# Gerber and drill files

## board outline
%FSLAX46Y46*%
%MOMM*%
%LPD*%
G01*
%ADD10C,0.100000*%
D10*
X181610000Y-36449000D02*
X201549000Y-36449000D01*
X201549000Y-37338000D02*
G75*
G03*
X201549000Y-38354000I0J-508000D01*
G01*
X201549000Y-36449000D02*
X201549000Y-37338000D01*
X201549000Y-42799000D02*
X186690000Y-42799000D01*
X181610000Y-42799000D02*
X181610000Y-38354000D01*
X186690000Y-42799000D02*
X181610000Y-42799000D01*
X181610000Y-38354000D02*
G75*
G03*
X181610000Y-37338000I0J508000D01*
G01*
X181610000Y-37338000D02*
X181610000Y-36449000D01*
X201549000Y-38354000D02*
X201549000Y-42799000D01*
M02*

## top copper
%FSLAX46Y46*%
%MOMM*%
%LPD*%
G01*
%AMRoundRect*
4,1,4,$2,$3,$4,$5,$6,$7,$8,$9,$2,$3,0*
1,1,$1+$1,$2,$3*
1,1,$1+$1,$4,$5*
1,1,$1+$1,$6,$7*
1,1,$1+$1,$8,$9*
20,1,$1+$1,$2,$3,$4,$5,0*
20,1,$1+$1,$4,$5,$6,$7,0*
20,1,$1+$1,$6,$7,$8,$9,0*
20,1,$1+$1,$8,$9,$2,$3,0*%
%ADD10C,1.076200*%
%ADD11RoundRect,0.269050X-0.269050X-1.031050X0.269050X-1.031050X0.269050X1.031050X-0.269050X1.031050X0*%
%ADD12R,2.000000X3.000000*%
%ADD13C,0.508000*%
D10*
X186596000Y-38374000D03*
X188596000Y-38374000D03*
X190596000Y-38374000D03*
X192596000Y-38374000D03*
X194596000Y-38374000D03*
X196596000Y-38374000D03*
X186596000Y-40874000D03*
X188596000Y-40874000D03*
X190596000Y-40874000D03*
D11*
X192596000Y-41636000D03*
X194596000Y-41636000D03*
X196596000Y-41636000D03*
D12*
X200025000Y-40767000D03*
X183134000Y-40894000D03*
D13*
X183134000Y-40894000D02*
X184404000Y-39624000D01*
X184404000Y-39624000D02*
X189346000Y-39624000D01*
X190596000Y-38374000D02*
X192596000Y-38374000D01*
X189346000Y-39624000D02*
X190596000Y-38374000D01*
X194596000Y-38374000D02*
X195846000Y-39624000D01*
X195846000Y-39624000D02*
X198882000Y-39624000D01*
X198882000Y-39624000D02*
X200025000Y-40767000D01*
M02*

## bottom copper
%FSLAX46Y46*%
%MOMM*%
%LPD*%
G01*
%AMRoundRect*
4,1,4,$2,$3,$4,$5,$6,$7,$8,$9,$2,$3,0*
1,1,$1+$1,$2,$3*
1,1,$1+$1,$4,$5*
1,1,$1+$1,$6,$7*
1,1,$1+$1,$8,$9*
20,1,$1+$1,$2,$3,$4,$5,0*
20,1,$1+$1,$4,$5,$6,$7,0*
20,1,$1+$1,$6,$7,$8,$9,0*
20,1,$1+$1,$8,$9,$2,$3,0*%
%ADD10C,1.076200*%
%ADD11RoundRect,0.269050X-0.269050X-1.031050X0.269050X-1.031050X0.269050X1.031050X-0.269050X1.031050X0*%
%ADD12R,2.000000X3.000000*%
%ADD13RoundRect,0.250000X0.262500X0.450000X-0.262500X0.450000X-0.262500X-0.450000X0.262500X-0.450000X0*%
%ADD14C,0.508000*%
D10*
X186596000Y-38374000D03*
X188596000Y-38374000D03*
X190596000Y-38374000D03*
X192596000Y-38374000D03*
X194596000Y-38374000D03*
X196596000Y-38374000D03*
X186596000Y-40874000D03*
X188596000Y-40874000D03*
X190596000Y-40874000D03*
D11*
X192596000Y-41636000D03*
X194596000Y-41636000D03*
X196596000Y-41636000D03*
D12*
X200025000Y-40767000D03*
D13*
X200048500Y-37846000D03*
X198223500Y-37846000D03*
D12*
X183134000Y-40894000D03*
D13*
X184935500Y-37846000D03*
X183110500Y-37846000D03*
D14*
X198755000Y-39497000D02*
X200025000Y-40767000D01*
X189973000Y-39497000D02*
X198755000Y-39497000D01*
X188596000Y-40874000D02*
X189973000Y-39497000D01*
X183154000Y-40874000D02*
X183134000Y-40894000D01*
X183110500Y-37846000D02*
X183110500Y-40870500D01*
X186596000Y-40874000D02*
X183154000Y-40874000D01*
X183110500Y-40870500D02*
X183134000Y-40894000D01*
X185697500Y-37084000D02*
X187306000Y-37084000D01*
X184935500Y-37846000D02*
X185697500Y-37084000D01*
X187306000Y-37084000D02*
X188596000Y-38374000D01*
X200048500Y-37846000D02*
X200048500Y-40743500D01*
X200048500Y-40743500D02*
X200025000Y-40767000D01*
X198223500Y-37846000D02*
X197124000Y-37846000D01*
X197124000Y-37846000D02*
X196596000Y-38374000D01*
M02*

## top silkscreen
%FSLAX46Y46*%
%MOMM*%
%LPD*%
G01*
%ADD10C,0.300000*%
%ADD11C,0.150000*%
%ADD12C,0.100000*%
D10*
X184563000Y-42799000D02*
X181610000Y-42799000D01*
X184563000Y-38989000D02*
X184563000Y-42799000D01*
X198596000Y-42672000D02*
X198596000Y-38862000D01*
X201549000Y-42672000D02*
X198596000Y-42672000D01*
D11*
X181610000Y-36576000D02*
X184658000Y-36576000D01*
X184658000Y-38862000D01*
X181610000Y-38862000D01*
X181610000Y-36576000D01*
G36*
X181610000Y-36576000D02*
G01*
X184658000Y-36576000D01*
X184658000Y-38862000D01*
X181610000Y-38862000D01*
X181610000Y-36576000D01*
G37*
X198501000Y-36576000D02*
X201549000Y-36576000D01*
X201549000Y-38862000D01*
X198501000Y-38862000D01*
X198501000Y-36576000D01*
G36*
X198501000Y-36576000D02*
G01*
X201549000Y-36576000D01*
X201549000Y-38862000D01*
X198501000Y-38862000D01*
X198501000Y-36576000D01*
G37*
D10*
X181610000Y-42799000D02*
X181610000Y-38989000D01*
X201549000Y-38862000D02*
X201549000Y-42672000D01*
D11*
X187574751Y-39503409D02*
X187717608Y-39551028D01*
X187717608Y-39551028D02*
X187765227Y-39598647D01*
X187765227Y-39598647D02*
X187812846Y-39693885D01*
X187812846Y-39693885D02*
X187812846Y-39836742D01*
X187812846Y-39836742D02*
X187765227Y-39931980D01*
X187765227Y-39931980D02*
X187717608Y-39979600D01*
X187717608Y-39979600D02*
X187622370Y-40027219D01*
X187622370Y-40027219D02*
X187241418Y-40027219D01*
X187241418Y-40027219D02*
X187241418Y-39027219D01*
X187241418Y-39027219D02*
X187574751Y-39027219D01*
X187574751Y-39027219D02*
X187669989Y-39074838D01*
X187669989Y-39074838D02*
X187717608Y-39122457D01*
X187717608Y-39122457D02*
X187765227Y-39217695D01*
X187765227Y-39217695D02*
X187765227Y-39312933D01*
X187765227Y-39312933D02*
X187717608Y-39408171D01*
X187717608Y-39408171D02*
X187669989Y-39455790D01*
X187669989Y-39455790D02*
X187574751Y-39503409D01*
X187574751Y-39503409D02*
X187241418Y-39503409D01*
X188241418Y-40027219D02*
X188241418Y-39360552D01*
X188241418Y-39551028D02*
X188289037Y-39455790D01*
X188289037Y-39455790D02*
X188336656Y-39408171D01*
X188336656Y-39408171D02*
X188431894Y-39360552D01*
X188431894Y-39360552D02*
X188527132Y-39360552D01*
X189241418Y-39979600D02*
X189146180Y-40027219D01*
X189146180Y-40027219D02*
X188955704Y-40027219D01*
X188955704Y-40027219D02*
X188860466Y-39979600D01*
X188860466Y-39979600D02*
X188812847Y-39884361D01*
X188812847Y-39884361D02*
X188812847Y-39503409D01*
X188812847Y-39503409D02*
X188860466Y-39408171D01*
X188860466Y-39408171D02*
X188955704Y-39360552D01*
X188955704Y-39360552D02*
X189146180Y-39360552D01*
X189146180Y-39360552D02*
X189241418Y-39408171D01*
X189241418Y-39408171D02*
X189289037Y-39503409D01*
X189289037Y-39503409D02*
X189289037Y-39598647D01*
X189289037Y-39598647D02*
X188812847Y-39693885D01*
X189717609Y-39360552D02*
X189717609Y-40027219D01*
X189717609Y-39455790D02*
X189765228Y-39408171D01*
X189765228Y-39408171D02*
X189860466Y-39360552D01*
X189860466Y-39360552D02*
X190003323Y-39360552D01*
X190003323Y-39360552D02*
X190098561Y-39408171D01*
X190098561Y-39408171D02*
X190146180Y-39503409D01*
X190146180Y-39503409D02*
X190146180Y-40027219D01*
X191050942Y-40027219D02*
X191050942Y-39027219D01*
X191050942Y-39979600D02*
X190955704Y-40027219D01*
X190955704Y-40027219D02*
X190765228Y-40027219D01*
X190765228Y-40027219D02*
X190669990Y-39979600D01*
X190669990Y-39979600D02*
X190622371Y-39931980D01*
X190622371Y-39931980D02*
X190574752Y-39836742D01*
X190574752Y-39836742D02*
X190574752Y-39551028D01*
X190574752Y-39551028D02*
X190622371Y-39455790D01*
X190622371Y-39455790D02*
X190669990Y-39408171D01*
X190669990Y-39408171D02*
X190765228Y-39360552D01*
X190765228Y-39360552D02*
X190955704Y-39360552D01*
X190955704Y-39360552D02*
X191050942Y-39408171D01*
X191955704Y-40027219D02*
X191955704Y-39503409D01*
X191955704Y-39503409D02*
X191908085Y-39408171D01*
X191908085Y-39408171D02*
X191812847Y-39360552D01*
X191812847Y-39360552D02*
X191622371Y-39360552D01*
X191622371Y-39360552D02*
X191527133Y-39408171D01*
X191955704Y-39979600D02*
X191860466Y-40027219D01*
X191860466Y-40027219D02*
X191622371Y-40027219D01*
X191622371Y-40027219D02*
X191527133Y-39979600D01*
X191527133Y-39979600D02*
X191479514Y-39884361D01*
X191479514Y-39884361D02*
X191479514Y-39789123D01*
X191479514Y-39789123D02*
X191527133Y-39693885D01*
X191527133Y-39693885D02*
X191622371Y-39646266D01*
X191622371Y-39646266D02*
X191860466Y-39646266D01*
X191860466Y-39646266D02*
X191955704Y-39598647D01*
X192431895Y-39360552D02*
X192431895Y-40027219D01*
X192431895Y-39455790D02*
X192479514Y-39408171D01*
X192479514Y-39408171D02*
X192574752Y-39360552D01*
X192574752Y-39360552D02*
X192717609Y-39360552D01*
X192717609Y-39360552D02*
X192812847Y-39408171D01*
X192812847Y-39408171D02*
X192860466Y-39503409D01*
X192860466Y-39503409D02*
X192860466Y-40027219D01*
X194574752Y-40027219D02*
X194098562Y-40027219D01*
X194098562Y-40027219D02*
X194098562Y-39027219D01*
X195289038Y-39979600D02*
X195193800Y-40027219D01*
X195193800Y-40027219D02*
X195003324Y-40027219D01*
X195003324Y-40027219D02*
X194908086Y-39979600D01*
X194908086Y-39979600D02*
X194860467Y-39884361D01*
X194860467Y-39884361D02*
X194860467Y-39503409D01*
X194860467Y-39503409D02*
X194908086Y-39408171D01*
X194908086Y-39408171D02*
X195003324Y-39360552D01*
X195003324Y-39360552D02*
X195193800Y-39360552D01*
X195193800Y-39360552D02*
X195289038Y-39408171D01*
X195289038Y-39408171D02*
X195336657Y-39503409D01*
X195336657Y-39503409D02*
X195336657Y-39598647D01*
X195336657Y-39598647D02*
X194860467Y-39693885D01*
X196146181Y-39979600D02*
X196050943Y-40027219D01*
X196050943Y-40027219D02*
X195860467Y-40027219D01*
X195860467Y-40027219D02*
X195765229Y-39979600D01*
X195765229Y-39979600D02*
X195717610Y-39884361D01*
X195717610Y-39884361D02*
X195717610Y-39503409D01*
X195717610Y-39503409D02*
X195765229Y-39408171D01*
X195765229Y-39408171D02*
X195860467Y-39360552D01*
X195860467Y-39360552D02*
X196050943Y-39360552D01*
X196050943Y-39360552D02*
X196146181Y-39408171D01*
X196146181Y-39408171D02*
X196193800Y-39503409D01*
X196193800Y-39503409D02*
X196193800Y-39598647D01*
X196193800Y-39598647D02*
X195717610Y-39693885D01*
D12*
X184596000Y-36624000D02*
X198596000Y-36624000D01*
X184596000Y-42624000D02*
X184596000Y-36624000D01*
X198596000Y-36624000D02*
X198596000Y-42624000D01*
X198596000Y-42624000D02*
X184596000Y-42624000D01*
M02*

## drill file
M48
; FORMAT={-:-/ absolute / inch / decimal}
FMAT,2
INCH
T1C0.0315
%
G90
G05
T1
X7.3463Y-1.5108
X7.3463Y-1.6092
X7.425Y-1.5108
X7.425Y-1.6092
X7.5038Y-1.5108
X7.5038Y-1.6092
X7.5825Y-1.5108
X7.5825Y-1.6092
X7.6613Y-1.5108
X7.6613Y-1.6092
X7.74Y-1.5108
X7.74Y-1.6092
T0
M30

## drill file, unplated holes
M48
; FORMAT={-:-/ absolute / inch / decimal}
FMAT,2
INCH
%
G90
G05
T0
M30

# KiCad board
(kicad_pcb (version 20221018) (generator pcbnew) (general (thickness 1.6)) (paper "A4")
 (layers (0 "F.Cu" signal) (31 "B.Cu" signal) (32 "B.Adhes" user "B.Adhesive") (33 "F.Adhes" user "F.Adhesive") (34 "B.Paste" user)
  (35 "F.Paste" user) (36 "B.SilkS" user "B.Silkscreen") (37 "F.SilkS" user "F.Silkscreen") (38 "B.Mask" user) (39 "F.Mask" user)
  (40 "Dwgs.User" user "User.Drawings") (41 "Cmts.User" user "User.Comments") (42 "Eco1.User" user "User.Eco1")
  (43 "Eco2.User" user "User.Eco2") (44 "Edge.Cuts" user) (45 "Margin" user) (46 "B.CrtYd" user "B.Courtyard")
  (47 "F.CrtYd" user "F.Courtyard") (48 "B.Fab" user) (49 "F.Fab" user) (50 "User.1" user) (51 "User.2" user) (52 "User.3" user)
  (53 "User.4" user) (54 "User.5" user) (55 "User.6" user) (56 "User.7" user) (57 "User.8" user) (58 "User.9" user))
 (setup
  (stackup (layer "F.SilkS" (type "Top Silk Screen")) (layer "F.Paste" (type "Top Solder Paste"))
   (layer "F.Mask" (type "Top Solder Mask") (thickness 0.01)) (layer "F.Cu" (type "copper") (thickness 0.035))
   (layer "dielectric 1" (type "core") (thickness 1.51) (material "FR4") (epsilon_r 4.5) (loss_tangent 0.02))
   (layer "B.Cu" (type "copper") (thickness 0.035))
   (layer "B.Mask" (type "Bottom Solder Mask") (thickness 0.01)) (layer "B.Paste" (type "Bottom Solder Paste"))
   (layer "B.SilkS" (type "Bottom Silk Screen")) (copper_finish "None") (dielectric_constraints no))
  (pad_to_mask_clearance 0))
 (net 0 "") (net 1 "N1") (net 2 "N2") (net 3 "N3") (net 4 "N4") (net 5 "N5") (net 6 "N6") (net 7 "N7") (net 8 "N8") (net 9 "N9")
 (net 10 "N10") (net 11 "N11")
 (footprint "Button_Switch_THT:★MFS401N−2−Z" (layer "F.Cu") (at 191.596 39.624)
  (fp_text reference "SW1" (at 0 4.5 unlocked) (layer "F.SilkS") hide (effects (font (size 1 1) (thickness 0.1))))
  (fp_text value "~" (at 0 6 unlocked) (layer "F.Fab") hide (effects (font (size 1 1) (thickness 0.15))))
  (fp_line (start -7 -3) (end 7 -3) (stroke (width 0.1) (type default)) (layer "F.SilkS"))
  (fp_line (start -7 3) (end -7 -3) (stroke (width 0.1) (type default)) (layer "F.SilkS"))
  (fp_line (start 7 -3) (end 7 3) (stroke (width 0.1) (type default)) (layer "F.SilkS"))
  (fp_line (start 7 3) (end -7 3) (stroke (width 0.1) (type default)) (layer "F.SilkS"))
  (pad "1" thru_hole circle (at -5 -1.25) (size 1.0762 1.0762) (drill 0.8) (layers "*.Cu" "*.Mask") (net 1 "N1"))
  (pad "2" thru_hole circle (at -3 -1.25) (size 1.0762 1.0762) (drill 0.8) (layers "*.Cu" "*.Mask") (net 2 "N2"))
  (pad "3" thru_hole circle (at -1 -1.25) (size 1.0762 1.0762) (drill 0.8) (layers "*.Cu" "*.Mask") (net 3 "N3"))
  (pad "4" thru_hole circle (at 1 -1.25) (size 1.0762 1.0762) (drill 0.8) (layers "*.Cu" "*.Mask") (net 3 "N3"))
  (pad "5" thru_hole circle (at 3 -1.25) (size 1.0762 1.0762) (drill 0.8) (layers "*.Cu" "*.Mask") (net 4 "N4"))
  (pad "6" thru_hole circle (at 5 -1.25) (size 1.0762 1.0762) (drill 0.8) (layers "*.Cu" "*.Mask") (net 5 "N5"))
  (pad "7" thru_hole circle (at -5 1.25) (size 1.0762 1.0762) (drill 0.8) (layers "*.Cu" "*.Mask") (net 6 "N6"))
  (pad "8" thru_hole circle (at -3 1.25) (size 1.0762 1.0762) (drill 0.8) (layers "*.Cu" "*.Mask") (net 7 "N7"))
  (pad "9" thru_hole circle (at -1 1.25) (size 1.0762 1.0762) (drill 0.8) (layers "*.Cu" "*.Mask") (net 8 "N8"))
  (pad "10" thru_hole roundrect (at 1 1.25) (size 1.0762 2.6002) (drill 0.8 (offset 0 0.762)) (layers "*.Cu" "*.Mask")
   (roundrect_rratio 0.25) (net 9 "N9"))
  (pad "11" thru_hole roundrect (at 3 1.25) (size 1.0762 2.6002) (drill 0.8 (offset 0 0.762)) (layers "*.Cu" "*.Mask")
   (roundrect_rratio 0.25) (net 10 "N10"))
  (pad "12" thru_hole roundrect (at 5 1.25) (size 1.0762 2.6002) (drill 0.8 (offset 0 0.762)) (layers "*.Cu" "*.Mask")
   (roundrect_rratio 0.25) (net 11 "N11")))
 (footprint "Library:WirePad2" (layer "B.Cu") (at 200.025 40.767)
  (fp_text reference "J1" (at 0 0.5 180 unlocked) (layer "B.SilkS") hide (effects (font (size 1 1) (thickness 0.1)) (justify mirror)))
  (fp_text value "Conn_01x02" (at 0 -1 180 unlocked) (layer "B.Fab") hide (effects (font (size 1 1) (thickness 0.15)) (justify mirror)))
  (pad "1" smd rect (at 0 0 180) (size 2 3) (layers "B.Cu" "B.Paste" "B.Mask") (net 7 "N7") (thermal_bridge_angle 45))
  (pad "2" smd rect (at 0 0 90) (size 3 2) (layers "F.Cu" "F.Paste" "F.Mask") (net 4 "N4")))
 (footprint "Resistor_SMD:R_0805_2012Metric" (layer "B.Cu") (at 199.136 37.846 180)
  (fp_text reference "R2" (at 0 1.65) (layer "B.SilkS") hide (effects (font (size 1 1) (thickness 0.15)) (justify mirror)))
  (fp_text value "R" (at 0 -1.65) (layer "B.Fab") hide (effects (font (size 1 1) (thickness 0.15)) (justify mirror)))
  (pad "1" smd roundrect (at -0.9125 0 180) (size 1.025 1.4) (layers "B.Cu" "B.Paste" "B.Mask") (roundrect_rratio 0.243902) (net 7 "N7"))
  (pad "2" smd roundrect (at 0.9125 0 180) (size 1.025 1.4) (layers "B.Cu" "B.Paste" "B.Mask") (roundrect_rratio 0.243902) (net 5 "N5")))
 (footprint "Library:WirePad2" (layer "B.Cu") (at 183.134 40.894)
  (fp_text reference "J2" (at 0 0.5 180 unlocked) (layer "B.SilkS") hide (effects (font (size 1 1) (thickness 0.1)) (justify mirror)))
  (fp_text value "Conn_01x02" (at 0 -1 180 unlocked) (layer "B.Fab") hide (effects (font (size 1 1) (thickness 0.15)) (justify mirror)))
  (pad "1" smd rect (at 0 0 180) (size 2 3) (layers "B.Cu" "B.Paste" "B.Mask") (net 6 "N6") (thermal_bridge_angle 45))
  (pad "2" smd rect (at 0 0 90) (size 3 2) (layers "F.Cu" "F.Paste" "F.Mask") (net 3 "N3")))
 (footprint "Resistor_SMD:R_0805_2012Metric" (layer "B.Cu") (at 184.023 37.846 180)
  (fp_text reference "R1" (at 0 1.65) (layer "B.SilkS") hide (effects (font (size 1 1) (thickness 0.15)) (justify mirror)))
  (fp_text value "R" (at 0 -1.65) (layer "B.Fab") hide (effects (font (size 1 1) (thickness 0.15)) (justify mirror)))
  (pad "1" smd roundrect (at -0.9125 0 180) (size 1.025 1.4) (layers "B.Cu" "B.Paste" "B.Mask") (roundrect_rratio 0.243902) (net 2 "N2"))
  (pad "2" smd roundrect (at 0.9125 0 180) (size 1.025 1.4) (layers "B.Cu" "B.Paste" "B.Mask") (roundrect_rratio 0.243902) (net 6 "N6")))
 (gr_line (start 184.563 42.799) (end 181.61 42.799) (stroke (width 0.3) (type solid)) (layer "F.SilkS"))
 (gr_line (start 184.563 38.989) (end 184.563 42.799) (stroke (width 0.3) (type solid)) (layer "F.SilkS"))
 (gr_line (start 198.596 42.672) (end 198.596 38.862) (stroke (width 0.3) (type solid)) (layer "F.SilkS"))
 (gr_line (start 201.549 42.672) (end 198.596 42.672) (stroke (width 0.3) (type solid)) (layer "F.SilkS"))
 (gr_rect (start 181.61 36.576) (end 184.658 38.862) (stroke (width 0.15) (type solid)) (fill solid) (layer "F.SilkS"))
 (gr_rect (start 198.501 36.576) (end 201.549 38.862) (stroke (width 0.15) (type solid)) (fill solid) (layer "F.SilkS"))
 (gr_line (start 181.61 42.799) (end 181.61 38.989) (stroke (width 0.3) (type solid)) (layer "F.SilkS"))
 (gr_line (start 201.549 38.862) (end 201.549 42.672) (stroke (width 0.3) (type solid)) (layer "F.SilkS"))
 (gr_line (start 181.61 36.449) (end 201.549 36.449) (stroke (width 0.1) (type default)) (layer "Edge.Cuts"))
 (gr_arc (start 201.549 38.354) (mid 201.041 37.846) (end 201.549 37.338) (stroke (width 0.1) (type default)) (layer "Edge.Cuts"))
 (gr_line (start 201.549 36.449) (end 201.549 37.338) (stroke (width 0.1) (type default)) (layer "Edge.Cuts"))
 (gr_line (start 201.549 42.799) (end 186.69 42.799) (stroke (width 0.1) (type default)) (layer "Edge.Cuts"))
 (gr_line (start 181.61 42.799) (end 181.61 38.354) (stroke (width 0.1) (type default)) (layer "Edge.Cuts"))
 (gr_line (start 186.69 42.799) (end 181.61 42.799) (stroke (width 0.1) (type default)) (layer "Edge.Cuts"))
 (gr_arc (start 181.61 37.338) (mid 182.118 37.846) (end 181.61 38.354) (stroke (width 0.1) (type default)) (layer "Edge.Cuts"))
 (gr_line (start 181.61 37.338) (end 181.61 36.449) (stroke (width 0.1) (type default)) (layer "Edge.Cuts"))
 (gr_line (start 201.549 38.354) (end 201.549 42.799) (stroke (width 0.1) (type default)) (layer "Edge.Cuts"))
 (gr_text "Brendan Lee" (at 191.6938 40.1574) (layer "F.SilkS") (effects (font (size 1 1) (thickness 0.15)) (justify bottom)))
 (segment (start 183.154 40.874) (end 183.134 40.894) (width 0.508) (layer "B.Cu") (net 6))
 (segment (start 183.1105 37.846) (end 183.1105 40.8705) (width 0.508) (layer "B.Cu") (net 6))
 (segment (start 186.596 40.874) (end 183.154 40.874) (width 0.508) (layer "B.Cu") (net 6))
 (segment (start 183.1105 40.8705) (end 183.134 40.894) (width 0.508) (layer "B.Cu") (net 6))
 (segment (start 183.134 40.894) (end 184.404 39.624) (width 0.508) (layer "F.Cu") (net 3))
 (segment (start 184.404 39.624) (end 189.346 39.624) (width 0.508) (layer "F.Cu") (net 3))
 (segment (start 190.596 38.374) (end 192.596 38.374) (width 0.508) (layer "F.Cu") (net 3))
 (segment (start 189.346 39.624) (end 190.596 38.374) (width 0.508) (layer "F.Cu") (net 3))
 (segment (start 185.6975 37.084) (end 187.306 37.084) (width 0.508) (layer "B.Cu") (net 2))
 (segment (start 184.9355 37.846) (end 185.6975 37.084) (width 0.508) (layer "B.Cu") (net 2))
 (segment (start 187.306 37.084) (end 188.596 38.374) (width 0.508) (layer "B.Cu") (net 2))
 (segment (start 194.596 38.374) (end 195.846 39.624) (width 0.508) (layer "F.Cu") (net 4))
 (segment (start 195.846 39.624) (end 198.882 39.624) (width 0.508) (layer "F.Cu") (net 4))
 (segment (start 198.882 39.624) (end 200.025 40.767) (width 0.508) (layer "F.Cu") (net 4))
 (segment (start 189.973 39.497) (end 198.755 39.497) (width 0.508) (layer "B.Cu") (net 7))
 (segment (start 200.0485 37.846) (end 200.0485 40.7435) (width 0.508) (layer "B.Cu") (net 7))
 (segment (start 188.596 40.874) (end 189.973 39.497) (width 0.508) (layer "B.Cu") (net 7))
 (segment (start 198.755 39.497) (end 200.025 40.767) (width 0.508) (layer "B.Cu") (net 7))
 (segment (start 200.0485 40.7435) (end 200.025 40.767) (width 0.508) (layer "B.Cu") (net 7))
 (segment (start 198.2235 37.846) (end 197.124 37.846) (width 0.508) (layer "B.Cu") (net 5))
 (segment (start 197.124 37.846) (end 196.596 38.374) (width 0.508) (layer "B.Cu") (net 5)))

